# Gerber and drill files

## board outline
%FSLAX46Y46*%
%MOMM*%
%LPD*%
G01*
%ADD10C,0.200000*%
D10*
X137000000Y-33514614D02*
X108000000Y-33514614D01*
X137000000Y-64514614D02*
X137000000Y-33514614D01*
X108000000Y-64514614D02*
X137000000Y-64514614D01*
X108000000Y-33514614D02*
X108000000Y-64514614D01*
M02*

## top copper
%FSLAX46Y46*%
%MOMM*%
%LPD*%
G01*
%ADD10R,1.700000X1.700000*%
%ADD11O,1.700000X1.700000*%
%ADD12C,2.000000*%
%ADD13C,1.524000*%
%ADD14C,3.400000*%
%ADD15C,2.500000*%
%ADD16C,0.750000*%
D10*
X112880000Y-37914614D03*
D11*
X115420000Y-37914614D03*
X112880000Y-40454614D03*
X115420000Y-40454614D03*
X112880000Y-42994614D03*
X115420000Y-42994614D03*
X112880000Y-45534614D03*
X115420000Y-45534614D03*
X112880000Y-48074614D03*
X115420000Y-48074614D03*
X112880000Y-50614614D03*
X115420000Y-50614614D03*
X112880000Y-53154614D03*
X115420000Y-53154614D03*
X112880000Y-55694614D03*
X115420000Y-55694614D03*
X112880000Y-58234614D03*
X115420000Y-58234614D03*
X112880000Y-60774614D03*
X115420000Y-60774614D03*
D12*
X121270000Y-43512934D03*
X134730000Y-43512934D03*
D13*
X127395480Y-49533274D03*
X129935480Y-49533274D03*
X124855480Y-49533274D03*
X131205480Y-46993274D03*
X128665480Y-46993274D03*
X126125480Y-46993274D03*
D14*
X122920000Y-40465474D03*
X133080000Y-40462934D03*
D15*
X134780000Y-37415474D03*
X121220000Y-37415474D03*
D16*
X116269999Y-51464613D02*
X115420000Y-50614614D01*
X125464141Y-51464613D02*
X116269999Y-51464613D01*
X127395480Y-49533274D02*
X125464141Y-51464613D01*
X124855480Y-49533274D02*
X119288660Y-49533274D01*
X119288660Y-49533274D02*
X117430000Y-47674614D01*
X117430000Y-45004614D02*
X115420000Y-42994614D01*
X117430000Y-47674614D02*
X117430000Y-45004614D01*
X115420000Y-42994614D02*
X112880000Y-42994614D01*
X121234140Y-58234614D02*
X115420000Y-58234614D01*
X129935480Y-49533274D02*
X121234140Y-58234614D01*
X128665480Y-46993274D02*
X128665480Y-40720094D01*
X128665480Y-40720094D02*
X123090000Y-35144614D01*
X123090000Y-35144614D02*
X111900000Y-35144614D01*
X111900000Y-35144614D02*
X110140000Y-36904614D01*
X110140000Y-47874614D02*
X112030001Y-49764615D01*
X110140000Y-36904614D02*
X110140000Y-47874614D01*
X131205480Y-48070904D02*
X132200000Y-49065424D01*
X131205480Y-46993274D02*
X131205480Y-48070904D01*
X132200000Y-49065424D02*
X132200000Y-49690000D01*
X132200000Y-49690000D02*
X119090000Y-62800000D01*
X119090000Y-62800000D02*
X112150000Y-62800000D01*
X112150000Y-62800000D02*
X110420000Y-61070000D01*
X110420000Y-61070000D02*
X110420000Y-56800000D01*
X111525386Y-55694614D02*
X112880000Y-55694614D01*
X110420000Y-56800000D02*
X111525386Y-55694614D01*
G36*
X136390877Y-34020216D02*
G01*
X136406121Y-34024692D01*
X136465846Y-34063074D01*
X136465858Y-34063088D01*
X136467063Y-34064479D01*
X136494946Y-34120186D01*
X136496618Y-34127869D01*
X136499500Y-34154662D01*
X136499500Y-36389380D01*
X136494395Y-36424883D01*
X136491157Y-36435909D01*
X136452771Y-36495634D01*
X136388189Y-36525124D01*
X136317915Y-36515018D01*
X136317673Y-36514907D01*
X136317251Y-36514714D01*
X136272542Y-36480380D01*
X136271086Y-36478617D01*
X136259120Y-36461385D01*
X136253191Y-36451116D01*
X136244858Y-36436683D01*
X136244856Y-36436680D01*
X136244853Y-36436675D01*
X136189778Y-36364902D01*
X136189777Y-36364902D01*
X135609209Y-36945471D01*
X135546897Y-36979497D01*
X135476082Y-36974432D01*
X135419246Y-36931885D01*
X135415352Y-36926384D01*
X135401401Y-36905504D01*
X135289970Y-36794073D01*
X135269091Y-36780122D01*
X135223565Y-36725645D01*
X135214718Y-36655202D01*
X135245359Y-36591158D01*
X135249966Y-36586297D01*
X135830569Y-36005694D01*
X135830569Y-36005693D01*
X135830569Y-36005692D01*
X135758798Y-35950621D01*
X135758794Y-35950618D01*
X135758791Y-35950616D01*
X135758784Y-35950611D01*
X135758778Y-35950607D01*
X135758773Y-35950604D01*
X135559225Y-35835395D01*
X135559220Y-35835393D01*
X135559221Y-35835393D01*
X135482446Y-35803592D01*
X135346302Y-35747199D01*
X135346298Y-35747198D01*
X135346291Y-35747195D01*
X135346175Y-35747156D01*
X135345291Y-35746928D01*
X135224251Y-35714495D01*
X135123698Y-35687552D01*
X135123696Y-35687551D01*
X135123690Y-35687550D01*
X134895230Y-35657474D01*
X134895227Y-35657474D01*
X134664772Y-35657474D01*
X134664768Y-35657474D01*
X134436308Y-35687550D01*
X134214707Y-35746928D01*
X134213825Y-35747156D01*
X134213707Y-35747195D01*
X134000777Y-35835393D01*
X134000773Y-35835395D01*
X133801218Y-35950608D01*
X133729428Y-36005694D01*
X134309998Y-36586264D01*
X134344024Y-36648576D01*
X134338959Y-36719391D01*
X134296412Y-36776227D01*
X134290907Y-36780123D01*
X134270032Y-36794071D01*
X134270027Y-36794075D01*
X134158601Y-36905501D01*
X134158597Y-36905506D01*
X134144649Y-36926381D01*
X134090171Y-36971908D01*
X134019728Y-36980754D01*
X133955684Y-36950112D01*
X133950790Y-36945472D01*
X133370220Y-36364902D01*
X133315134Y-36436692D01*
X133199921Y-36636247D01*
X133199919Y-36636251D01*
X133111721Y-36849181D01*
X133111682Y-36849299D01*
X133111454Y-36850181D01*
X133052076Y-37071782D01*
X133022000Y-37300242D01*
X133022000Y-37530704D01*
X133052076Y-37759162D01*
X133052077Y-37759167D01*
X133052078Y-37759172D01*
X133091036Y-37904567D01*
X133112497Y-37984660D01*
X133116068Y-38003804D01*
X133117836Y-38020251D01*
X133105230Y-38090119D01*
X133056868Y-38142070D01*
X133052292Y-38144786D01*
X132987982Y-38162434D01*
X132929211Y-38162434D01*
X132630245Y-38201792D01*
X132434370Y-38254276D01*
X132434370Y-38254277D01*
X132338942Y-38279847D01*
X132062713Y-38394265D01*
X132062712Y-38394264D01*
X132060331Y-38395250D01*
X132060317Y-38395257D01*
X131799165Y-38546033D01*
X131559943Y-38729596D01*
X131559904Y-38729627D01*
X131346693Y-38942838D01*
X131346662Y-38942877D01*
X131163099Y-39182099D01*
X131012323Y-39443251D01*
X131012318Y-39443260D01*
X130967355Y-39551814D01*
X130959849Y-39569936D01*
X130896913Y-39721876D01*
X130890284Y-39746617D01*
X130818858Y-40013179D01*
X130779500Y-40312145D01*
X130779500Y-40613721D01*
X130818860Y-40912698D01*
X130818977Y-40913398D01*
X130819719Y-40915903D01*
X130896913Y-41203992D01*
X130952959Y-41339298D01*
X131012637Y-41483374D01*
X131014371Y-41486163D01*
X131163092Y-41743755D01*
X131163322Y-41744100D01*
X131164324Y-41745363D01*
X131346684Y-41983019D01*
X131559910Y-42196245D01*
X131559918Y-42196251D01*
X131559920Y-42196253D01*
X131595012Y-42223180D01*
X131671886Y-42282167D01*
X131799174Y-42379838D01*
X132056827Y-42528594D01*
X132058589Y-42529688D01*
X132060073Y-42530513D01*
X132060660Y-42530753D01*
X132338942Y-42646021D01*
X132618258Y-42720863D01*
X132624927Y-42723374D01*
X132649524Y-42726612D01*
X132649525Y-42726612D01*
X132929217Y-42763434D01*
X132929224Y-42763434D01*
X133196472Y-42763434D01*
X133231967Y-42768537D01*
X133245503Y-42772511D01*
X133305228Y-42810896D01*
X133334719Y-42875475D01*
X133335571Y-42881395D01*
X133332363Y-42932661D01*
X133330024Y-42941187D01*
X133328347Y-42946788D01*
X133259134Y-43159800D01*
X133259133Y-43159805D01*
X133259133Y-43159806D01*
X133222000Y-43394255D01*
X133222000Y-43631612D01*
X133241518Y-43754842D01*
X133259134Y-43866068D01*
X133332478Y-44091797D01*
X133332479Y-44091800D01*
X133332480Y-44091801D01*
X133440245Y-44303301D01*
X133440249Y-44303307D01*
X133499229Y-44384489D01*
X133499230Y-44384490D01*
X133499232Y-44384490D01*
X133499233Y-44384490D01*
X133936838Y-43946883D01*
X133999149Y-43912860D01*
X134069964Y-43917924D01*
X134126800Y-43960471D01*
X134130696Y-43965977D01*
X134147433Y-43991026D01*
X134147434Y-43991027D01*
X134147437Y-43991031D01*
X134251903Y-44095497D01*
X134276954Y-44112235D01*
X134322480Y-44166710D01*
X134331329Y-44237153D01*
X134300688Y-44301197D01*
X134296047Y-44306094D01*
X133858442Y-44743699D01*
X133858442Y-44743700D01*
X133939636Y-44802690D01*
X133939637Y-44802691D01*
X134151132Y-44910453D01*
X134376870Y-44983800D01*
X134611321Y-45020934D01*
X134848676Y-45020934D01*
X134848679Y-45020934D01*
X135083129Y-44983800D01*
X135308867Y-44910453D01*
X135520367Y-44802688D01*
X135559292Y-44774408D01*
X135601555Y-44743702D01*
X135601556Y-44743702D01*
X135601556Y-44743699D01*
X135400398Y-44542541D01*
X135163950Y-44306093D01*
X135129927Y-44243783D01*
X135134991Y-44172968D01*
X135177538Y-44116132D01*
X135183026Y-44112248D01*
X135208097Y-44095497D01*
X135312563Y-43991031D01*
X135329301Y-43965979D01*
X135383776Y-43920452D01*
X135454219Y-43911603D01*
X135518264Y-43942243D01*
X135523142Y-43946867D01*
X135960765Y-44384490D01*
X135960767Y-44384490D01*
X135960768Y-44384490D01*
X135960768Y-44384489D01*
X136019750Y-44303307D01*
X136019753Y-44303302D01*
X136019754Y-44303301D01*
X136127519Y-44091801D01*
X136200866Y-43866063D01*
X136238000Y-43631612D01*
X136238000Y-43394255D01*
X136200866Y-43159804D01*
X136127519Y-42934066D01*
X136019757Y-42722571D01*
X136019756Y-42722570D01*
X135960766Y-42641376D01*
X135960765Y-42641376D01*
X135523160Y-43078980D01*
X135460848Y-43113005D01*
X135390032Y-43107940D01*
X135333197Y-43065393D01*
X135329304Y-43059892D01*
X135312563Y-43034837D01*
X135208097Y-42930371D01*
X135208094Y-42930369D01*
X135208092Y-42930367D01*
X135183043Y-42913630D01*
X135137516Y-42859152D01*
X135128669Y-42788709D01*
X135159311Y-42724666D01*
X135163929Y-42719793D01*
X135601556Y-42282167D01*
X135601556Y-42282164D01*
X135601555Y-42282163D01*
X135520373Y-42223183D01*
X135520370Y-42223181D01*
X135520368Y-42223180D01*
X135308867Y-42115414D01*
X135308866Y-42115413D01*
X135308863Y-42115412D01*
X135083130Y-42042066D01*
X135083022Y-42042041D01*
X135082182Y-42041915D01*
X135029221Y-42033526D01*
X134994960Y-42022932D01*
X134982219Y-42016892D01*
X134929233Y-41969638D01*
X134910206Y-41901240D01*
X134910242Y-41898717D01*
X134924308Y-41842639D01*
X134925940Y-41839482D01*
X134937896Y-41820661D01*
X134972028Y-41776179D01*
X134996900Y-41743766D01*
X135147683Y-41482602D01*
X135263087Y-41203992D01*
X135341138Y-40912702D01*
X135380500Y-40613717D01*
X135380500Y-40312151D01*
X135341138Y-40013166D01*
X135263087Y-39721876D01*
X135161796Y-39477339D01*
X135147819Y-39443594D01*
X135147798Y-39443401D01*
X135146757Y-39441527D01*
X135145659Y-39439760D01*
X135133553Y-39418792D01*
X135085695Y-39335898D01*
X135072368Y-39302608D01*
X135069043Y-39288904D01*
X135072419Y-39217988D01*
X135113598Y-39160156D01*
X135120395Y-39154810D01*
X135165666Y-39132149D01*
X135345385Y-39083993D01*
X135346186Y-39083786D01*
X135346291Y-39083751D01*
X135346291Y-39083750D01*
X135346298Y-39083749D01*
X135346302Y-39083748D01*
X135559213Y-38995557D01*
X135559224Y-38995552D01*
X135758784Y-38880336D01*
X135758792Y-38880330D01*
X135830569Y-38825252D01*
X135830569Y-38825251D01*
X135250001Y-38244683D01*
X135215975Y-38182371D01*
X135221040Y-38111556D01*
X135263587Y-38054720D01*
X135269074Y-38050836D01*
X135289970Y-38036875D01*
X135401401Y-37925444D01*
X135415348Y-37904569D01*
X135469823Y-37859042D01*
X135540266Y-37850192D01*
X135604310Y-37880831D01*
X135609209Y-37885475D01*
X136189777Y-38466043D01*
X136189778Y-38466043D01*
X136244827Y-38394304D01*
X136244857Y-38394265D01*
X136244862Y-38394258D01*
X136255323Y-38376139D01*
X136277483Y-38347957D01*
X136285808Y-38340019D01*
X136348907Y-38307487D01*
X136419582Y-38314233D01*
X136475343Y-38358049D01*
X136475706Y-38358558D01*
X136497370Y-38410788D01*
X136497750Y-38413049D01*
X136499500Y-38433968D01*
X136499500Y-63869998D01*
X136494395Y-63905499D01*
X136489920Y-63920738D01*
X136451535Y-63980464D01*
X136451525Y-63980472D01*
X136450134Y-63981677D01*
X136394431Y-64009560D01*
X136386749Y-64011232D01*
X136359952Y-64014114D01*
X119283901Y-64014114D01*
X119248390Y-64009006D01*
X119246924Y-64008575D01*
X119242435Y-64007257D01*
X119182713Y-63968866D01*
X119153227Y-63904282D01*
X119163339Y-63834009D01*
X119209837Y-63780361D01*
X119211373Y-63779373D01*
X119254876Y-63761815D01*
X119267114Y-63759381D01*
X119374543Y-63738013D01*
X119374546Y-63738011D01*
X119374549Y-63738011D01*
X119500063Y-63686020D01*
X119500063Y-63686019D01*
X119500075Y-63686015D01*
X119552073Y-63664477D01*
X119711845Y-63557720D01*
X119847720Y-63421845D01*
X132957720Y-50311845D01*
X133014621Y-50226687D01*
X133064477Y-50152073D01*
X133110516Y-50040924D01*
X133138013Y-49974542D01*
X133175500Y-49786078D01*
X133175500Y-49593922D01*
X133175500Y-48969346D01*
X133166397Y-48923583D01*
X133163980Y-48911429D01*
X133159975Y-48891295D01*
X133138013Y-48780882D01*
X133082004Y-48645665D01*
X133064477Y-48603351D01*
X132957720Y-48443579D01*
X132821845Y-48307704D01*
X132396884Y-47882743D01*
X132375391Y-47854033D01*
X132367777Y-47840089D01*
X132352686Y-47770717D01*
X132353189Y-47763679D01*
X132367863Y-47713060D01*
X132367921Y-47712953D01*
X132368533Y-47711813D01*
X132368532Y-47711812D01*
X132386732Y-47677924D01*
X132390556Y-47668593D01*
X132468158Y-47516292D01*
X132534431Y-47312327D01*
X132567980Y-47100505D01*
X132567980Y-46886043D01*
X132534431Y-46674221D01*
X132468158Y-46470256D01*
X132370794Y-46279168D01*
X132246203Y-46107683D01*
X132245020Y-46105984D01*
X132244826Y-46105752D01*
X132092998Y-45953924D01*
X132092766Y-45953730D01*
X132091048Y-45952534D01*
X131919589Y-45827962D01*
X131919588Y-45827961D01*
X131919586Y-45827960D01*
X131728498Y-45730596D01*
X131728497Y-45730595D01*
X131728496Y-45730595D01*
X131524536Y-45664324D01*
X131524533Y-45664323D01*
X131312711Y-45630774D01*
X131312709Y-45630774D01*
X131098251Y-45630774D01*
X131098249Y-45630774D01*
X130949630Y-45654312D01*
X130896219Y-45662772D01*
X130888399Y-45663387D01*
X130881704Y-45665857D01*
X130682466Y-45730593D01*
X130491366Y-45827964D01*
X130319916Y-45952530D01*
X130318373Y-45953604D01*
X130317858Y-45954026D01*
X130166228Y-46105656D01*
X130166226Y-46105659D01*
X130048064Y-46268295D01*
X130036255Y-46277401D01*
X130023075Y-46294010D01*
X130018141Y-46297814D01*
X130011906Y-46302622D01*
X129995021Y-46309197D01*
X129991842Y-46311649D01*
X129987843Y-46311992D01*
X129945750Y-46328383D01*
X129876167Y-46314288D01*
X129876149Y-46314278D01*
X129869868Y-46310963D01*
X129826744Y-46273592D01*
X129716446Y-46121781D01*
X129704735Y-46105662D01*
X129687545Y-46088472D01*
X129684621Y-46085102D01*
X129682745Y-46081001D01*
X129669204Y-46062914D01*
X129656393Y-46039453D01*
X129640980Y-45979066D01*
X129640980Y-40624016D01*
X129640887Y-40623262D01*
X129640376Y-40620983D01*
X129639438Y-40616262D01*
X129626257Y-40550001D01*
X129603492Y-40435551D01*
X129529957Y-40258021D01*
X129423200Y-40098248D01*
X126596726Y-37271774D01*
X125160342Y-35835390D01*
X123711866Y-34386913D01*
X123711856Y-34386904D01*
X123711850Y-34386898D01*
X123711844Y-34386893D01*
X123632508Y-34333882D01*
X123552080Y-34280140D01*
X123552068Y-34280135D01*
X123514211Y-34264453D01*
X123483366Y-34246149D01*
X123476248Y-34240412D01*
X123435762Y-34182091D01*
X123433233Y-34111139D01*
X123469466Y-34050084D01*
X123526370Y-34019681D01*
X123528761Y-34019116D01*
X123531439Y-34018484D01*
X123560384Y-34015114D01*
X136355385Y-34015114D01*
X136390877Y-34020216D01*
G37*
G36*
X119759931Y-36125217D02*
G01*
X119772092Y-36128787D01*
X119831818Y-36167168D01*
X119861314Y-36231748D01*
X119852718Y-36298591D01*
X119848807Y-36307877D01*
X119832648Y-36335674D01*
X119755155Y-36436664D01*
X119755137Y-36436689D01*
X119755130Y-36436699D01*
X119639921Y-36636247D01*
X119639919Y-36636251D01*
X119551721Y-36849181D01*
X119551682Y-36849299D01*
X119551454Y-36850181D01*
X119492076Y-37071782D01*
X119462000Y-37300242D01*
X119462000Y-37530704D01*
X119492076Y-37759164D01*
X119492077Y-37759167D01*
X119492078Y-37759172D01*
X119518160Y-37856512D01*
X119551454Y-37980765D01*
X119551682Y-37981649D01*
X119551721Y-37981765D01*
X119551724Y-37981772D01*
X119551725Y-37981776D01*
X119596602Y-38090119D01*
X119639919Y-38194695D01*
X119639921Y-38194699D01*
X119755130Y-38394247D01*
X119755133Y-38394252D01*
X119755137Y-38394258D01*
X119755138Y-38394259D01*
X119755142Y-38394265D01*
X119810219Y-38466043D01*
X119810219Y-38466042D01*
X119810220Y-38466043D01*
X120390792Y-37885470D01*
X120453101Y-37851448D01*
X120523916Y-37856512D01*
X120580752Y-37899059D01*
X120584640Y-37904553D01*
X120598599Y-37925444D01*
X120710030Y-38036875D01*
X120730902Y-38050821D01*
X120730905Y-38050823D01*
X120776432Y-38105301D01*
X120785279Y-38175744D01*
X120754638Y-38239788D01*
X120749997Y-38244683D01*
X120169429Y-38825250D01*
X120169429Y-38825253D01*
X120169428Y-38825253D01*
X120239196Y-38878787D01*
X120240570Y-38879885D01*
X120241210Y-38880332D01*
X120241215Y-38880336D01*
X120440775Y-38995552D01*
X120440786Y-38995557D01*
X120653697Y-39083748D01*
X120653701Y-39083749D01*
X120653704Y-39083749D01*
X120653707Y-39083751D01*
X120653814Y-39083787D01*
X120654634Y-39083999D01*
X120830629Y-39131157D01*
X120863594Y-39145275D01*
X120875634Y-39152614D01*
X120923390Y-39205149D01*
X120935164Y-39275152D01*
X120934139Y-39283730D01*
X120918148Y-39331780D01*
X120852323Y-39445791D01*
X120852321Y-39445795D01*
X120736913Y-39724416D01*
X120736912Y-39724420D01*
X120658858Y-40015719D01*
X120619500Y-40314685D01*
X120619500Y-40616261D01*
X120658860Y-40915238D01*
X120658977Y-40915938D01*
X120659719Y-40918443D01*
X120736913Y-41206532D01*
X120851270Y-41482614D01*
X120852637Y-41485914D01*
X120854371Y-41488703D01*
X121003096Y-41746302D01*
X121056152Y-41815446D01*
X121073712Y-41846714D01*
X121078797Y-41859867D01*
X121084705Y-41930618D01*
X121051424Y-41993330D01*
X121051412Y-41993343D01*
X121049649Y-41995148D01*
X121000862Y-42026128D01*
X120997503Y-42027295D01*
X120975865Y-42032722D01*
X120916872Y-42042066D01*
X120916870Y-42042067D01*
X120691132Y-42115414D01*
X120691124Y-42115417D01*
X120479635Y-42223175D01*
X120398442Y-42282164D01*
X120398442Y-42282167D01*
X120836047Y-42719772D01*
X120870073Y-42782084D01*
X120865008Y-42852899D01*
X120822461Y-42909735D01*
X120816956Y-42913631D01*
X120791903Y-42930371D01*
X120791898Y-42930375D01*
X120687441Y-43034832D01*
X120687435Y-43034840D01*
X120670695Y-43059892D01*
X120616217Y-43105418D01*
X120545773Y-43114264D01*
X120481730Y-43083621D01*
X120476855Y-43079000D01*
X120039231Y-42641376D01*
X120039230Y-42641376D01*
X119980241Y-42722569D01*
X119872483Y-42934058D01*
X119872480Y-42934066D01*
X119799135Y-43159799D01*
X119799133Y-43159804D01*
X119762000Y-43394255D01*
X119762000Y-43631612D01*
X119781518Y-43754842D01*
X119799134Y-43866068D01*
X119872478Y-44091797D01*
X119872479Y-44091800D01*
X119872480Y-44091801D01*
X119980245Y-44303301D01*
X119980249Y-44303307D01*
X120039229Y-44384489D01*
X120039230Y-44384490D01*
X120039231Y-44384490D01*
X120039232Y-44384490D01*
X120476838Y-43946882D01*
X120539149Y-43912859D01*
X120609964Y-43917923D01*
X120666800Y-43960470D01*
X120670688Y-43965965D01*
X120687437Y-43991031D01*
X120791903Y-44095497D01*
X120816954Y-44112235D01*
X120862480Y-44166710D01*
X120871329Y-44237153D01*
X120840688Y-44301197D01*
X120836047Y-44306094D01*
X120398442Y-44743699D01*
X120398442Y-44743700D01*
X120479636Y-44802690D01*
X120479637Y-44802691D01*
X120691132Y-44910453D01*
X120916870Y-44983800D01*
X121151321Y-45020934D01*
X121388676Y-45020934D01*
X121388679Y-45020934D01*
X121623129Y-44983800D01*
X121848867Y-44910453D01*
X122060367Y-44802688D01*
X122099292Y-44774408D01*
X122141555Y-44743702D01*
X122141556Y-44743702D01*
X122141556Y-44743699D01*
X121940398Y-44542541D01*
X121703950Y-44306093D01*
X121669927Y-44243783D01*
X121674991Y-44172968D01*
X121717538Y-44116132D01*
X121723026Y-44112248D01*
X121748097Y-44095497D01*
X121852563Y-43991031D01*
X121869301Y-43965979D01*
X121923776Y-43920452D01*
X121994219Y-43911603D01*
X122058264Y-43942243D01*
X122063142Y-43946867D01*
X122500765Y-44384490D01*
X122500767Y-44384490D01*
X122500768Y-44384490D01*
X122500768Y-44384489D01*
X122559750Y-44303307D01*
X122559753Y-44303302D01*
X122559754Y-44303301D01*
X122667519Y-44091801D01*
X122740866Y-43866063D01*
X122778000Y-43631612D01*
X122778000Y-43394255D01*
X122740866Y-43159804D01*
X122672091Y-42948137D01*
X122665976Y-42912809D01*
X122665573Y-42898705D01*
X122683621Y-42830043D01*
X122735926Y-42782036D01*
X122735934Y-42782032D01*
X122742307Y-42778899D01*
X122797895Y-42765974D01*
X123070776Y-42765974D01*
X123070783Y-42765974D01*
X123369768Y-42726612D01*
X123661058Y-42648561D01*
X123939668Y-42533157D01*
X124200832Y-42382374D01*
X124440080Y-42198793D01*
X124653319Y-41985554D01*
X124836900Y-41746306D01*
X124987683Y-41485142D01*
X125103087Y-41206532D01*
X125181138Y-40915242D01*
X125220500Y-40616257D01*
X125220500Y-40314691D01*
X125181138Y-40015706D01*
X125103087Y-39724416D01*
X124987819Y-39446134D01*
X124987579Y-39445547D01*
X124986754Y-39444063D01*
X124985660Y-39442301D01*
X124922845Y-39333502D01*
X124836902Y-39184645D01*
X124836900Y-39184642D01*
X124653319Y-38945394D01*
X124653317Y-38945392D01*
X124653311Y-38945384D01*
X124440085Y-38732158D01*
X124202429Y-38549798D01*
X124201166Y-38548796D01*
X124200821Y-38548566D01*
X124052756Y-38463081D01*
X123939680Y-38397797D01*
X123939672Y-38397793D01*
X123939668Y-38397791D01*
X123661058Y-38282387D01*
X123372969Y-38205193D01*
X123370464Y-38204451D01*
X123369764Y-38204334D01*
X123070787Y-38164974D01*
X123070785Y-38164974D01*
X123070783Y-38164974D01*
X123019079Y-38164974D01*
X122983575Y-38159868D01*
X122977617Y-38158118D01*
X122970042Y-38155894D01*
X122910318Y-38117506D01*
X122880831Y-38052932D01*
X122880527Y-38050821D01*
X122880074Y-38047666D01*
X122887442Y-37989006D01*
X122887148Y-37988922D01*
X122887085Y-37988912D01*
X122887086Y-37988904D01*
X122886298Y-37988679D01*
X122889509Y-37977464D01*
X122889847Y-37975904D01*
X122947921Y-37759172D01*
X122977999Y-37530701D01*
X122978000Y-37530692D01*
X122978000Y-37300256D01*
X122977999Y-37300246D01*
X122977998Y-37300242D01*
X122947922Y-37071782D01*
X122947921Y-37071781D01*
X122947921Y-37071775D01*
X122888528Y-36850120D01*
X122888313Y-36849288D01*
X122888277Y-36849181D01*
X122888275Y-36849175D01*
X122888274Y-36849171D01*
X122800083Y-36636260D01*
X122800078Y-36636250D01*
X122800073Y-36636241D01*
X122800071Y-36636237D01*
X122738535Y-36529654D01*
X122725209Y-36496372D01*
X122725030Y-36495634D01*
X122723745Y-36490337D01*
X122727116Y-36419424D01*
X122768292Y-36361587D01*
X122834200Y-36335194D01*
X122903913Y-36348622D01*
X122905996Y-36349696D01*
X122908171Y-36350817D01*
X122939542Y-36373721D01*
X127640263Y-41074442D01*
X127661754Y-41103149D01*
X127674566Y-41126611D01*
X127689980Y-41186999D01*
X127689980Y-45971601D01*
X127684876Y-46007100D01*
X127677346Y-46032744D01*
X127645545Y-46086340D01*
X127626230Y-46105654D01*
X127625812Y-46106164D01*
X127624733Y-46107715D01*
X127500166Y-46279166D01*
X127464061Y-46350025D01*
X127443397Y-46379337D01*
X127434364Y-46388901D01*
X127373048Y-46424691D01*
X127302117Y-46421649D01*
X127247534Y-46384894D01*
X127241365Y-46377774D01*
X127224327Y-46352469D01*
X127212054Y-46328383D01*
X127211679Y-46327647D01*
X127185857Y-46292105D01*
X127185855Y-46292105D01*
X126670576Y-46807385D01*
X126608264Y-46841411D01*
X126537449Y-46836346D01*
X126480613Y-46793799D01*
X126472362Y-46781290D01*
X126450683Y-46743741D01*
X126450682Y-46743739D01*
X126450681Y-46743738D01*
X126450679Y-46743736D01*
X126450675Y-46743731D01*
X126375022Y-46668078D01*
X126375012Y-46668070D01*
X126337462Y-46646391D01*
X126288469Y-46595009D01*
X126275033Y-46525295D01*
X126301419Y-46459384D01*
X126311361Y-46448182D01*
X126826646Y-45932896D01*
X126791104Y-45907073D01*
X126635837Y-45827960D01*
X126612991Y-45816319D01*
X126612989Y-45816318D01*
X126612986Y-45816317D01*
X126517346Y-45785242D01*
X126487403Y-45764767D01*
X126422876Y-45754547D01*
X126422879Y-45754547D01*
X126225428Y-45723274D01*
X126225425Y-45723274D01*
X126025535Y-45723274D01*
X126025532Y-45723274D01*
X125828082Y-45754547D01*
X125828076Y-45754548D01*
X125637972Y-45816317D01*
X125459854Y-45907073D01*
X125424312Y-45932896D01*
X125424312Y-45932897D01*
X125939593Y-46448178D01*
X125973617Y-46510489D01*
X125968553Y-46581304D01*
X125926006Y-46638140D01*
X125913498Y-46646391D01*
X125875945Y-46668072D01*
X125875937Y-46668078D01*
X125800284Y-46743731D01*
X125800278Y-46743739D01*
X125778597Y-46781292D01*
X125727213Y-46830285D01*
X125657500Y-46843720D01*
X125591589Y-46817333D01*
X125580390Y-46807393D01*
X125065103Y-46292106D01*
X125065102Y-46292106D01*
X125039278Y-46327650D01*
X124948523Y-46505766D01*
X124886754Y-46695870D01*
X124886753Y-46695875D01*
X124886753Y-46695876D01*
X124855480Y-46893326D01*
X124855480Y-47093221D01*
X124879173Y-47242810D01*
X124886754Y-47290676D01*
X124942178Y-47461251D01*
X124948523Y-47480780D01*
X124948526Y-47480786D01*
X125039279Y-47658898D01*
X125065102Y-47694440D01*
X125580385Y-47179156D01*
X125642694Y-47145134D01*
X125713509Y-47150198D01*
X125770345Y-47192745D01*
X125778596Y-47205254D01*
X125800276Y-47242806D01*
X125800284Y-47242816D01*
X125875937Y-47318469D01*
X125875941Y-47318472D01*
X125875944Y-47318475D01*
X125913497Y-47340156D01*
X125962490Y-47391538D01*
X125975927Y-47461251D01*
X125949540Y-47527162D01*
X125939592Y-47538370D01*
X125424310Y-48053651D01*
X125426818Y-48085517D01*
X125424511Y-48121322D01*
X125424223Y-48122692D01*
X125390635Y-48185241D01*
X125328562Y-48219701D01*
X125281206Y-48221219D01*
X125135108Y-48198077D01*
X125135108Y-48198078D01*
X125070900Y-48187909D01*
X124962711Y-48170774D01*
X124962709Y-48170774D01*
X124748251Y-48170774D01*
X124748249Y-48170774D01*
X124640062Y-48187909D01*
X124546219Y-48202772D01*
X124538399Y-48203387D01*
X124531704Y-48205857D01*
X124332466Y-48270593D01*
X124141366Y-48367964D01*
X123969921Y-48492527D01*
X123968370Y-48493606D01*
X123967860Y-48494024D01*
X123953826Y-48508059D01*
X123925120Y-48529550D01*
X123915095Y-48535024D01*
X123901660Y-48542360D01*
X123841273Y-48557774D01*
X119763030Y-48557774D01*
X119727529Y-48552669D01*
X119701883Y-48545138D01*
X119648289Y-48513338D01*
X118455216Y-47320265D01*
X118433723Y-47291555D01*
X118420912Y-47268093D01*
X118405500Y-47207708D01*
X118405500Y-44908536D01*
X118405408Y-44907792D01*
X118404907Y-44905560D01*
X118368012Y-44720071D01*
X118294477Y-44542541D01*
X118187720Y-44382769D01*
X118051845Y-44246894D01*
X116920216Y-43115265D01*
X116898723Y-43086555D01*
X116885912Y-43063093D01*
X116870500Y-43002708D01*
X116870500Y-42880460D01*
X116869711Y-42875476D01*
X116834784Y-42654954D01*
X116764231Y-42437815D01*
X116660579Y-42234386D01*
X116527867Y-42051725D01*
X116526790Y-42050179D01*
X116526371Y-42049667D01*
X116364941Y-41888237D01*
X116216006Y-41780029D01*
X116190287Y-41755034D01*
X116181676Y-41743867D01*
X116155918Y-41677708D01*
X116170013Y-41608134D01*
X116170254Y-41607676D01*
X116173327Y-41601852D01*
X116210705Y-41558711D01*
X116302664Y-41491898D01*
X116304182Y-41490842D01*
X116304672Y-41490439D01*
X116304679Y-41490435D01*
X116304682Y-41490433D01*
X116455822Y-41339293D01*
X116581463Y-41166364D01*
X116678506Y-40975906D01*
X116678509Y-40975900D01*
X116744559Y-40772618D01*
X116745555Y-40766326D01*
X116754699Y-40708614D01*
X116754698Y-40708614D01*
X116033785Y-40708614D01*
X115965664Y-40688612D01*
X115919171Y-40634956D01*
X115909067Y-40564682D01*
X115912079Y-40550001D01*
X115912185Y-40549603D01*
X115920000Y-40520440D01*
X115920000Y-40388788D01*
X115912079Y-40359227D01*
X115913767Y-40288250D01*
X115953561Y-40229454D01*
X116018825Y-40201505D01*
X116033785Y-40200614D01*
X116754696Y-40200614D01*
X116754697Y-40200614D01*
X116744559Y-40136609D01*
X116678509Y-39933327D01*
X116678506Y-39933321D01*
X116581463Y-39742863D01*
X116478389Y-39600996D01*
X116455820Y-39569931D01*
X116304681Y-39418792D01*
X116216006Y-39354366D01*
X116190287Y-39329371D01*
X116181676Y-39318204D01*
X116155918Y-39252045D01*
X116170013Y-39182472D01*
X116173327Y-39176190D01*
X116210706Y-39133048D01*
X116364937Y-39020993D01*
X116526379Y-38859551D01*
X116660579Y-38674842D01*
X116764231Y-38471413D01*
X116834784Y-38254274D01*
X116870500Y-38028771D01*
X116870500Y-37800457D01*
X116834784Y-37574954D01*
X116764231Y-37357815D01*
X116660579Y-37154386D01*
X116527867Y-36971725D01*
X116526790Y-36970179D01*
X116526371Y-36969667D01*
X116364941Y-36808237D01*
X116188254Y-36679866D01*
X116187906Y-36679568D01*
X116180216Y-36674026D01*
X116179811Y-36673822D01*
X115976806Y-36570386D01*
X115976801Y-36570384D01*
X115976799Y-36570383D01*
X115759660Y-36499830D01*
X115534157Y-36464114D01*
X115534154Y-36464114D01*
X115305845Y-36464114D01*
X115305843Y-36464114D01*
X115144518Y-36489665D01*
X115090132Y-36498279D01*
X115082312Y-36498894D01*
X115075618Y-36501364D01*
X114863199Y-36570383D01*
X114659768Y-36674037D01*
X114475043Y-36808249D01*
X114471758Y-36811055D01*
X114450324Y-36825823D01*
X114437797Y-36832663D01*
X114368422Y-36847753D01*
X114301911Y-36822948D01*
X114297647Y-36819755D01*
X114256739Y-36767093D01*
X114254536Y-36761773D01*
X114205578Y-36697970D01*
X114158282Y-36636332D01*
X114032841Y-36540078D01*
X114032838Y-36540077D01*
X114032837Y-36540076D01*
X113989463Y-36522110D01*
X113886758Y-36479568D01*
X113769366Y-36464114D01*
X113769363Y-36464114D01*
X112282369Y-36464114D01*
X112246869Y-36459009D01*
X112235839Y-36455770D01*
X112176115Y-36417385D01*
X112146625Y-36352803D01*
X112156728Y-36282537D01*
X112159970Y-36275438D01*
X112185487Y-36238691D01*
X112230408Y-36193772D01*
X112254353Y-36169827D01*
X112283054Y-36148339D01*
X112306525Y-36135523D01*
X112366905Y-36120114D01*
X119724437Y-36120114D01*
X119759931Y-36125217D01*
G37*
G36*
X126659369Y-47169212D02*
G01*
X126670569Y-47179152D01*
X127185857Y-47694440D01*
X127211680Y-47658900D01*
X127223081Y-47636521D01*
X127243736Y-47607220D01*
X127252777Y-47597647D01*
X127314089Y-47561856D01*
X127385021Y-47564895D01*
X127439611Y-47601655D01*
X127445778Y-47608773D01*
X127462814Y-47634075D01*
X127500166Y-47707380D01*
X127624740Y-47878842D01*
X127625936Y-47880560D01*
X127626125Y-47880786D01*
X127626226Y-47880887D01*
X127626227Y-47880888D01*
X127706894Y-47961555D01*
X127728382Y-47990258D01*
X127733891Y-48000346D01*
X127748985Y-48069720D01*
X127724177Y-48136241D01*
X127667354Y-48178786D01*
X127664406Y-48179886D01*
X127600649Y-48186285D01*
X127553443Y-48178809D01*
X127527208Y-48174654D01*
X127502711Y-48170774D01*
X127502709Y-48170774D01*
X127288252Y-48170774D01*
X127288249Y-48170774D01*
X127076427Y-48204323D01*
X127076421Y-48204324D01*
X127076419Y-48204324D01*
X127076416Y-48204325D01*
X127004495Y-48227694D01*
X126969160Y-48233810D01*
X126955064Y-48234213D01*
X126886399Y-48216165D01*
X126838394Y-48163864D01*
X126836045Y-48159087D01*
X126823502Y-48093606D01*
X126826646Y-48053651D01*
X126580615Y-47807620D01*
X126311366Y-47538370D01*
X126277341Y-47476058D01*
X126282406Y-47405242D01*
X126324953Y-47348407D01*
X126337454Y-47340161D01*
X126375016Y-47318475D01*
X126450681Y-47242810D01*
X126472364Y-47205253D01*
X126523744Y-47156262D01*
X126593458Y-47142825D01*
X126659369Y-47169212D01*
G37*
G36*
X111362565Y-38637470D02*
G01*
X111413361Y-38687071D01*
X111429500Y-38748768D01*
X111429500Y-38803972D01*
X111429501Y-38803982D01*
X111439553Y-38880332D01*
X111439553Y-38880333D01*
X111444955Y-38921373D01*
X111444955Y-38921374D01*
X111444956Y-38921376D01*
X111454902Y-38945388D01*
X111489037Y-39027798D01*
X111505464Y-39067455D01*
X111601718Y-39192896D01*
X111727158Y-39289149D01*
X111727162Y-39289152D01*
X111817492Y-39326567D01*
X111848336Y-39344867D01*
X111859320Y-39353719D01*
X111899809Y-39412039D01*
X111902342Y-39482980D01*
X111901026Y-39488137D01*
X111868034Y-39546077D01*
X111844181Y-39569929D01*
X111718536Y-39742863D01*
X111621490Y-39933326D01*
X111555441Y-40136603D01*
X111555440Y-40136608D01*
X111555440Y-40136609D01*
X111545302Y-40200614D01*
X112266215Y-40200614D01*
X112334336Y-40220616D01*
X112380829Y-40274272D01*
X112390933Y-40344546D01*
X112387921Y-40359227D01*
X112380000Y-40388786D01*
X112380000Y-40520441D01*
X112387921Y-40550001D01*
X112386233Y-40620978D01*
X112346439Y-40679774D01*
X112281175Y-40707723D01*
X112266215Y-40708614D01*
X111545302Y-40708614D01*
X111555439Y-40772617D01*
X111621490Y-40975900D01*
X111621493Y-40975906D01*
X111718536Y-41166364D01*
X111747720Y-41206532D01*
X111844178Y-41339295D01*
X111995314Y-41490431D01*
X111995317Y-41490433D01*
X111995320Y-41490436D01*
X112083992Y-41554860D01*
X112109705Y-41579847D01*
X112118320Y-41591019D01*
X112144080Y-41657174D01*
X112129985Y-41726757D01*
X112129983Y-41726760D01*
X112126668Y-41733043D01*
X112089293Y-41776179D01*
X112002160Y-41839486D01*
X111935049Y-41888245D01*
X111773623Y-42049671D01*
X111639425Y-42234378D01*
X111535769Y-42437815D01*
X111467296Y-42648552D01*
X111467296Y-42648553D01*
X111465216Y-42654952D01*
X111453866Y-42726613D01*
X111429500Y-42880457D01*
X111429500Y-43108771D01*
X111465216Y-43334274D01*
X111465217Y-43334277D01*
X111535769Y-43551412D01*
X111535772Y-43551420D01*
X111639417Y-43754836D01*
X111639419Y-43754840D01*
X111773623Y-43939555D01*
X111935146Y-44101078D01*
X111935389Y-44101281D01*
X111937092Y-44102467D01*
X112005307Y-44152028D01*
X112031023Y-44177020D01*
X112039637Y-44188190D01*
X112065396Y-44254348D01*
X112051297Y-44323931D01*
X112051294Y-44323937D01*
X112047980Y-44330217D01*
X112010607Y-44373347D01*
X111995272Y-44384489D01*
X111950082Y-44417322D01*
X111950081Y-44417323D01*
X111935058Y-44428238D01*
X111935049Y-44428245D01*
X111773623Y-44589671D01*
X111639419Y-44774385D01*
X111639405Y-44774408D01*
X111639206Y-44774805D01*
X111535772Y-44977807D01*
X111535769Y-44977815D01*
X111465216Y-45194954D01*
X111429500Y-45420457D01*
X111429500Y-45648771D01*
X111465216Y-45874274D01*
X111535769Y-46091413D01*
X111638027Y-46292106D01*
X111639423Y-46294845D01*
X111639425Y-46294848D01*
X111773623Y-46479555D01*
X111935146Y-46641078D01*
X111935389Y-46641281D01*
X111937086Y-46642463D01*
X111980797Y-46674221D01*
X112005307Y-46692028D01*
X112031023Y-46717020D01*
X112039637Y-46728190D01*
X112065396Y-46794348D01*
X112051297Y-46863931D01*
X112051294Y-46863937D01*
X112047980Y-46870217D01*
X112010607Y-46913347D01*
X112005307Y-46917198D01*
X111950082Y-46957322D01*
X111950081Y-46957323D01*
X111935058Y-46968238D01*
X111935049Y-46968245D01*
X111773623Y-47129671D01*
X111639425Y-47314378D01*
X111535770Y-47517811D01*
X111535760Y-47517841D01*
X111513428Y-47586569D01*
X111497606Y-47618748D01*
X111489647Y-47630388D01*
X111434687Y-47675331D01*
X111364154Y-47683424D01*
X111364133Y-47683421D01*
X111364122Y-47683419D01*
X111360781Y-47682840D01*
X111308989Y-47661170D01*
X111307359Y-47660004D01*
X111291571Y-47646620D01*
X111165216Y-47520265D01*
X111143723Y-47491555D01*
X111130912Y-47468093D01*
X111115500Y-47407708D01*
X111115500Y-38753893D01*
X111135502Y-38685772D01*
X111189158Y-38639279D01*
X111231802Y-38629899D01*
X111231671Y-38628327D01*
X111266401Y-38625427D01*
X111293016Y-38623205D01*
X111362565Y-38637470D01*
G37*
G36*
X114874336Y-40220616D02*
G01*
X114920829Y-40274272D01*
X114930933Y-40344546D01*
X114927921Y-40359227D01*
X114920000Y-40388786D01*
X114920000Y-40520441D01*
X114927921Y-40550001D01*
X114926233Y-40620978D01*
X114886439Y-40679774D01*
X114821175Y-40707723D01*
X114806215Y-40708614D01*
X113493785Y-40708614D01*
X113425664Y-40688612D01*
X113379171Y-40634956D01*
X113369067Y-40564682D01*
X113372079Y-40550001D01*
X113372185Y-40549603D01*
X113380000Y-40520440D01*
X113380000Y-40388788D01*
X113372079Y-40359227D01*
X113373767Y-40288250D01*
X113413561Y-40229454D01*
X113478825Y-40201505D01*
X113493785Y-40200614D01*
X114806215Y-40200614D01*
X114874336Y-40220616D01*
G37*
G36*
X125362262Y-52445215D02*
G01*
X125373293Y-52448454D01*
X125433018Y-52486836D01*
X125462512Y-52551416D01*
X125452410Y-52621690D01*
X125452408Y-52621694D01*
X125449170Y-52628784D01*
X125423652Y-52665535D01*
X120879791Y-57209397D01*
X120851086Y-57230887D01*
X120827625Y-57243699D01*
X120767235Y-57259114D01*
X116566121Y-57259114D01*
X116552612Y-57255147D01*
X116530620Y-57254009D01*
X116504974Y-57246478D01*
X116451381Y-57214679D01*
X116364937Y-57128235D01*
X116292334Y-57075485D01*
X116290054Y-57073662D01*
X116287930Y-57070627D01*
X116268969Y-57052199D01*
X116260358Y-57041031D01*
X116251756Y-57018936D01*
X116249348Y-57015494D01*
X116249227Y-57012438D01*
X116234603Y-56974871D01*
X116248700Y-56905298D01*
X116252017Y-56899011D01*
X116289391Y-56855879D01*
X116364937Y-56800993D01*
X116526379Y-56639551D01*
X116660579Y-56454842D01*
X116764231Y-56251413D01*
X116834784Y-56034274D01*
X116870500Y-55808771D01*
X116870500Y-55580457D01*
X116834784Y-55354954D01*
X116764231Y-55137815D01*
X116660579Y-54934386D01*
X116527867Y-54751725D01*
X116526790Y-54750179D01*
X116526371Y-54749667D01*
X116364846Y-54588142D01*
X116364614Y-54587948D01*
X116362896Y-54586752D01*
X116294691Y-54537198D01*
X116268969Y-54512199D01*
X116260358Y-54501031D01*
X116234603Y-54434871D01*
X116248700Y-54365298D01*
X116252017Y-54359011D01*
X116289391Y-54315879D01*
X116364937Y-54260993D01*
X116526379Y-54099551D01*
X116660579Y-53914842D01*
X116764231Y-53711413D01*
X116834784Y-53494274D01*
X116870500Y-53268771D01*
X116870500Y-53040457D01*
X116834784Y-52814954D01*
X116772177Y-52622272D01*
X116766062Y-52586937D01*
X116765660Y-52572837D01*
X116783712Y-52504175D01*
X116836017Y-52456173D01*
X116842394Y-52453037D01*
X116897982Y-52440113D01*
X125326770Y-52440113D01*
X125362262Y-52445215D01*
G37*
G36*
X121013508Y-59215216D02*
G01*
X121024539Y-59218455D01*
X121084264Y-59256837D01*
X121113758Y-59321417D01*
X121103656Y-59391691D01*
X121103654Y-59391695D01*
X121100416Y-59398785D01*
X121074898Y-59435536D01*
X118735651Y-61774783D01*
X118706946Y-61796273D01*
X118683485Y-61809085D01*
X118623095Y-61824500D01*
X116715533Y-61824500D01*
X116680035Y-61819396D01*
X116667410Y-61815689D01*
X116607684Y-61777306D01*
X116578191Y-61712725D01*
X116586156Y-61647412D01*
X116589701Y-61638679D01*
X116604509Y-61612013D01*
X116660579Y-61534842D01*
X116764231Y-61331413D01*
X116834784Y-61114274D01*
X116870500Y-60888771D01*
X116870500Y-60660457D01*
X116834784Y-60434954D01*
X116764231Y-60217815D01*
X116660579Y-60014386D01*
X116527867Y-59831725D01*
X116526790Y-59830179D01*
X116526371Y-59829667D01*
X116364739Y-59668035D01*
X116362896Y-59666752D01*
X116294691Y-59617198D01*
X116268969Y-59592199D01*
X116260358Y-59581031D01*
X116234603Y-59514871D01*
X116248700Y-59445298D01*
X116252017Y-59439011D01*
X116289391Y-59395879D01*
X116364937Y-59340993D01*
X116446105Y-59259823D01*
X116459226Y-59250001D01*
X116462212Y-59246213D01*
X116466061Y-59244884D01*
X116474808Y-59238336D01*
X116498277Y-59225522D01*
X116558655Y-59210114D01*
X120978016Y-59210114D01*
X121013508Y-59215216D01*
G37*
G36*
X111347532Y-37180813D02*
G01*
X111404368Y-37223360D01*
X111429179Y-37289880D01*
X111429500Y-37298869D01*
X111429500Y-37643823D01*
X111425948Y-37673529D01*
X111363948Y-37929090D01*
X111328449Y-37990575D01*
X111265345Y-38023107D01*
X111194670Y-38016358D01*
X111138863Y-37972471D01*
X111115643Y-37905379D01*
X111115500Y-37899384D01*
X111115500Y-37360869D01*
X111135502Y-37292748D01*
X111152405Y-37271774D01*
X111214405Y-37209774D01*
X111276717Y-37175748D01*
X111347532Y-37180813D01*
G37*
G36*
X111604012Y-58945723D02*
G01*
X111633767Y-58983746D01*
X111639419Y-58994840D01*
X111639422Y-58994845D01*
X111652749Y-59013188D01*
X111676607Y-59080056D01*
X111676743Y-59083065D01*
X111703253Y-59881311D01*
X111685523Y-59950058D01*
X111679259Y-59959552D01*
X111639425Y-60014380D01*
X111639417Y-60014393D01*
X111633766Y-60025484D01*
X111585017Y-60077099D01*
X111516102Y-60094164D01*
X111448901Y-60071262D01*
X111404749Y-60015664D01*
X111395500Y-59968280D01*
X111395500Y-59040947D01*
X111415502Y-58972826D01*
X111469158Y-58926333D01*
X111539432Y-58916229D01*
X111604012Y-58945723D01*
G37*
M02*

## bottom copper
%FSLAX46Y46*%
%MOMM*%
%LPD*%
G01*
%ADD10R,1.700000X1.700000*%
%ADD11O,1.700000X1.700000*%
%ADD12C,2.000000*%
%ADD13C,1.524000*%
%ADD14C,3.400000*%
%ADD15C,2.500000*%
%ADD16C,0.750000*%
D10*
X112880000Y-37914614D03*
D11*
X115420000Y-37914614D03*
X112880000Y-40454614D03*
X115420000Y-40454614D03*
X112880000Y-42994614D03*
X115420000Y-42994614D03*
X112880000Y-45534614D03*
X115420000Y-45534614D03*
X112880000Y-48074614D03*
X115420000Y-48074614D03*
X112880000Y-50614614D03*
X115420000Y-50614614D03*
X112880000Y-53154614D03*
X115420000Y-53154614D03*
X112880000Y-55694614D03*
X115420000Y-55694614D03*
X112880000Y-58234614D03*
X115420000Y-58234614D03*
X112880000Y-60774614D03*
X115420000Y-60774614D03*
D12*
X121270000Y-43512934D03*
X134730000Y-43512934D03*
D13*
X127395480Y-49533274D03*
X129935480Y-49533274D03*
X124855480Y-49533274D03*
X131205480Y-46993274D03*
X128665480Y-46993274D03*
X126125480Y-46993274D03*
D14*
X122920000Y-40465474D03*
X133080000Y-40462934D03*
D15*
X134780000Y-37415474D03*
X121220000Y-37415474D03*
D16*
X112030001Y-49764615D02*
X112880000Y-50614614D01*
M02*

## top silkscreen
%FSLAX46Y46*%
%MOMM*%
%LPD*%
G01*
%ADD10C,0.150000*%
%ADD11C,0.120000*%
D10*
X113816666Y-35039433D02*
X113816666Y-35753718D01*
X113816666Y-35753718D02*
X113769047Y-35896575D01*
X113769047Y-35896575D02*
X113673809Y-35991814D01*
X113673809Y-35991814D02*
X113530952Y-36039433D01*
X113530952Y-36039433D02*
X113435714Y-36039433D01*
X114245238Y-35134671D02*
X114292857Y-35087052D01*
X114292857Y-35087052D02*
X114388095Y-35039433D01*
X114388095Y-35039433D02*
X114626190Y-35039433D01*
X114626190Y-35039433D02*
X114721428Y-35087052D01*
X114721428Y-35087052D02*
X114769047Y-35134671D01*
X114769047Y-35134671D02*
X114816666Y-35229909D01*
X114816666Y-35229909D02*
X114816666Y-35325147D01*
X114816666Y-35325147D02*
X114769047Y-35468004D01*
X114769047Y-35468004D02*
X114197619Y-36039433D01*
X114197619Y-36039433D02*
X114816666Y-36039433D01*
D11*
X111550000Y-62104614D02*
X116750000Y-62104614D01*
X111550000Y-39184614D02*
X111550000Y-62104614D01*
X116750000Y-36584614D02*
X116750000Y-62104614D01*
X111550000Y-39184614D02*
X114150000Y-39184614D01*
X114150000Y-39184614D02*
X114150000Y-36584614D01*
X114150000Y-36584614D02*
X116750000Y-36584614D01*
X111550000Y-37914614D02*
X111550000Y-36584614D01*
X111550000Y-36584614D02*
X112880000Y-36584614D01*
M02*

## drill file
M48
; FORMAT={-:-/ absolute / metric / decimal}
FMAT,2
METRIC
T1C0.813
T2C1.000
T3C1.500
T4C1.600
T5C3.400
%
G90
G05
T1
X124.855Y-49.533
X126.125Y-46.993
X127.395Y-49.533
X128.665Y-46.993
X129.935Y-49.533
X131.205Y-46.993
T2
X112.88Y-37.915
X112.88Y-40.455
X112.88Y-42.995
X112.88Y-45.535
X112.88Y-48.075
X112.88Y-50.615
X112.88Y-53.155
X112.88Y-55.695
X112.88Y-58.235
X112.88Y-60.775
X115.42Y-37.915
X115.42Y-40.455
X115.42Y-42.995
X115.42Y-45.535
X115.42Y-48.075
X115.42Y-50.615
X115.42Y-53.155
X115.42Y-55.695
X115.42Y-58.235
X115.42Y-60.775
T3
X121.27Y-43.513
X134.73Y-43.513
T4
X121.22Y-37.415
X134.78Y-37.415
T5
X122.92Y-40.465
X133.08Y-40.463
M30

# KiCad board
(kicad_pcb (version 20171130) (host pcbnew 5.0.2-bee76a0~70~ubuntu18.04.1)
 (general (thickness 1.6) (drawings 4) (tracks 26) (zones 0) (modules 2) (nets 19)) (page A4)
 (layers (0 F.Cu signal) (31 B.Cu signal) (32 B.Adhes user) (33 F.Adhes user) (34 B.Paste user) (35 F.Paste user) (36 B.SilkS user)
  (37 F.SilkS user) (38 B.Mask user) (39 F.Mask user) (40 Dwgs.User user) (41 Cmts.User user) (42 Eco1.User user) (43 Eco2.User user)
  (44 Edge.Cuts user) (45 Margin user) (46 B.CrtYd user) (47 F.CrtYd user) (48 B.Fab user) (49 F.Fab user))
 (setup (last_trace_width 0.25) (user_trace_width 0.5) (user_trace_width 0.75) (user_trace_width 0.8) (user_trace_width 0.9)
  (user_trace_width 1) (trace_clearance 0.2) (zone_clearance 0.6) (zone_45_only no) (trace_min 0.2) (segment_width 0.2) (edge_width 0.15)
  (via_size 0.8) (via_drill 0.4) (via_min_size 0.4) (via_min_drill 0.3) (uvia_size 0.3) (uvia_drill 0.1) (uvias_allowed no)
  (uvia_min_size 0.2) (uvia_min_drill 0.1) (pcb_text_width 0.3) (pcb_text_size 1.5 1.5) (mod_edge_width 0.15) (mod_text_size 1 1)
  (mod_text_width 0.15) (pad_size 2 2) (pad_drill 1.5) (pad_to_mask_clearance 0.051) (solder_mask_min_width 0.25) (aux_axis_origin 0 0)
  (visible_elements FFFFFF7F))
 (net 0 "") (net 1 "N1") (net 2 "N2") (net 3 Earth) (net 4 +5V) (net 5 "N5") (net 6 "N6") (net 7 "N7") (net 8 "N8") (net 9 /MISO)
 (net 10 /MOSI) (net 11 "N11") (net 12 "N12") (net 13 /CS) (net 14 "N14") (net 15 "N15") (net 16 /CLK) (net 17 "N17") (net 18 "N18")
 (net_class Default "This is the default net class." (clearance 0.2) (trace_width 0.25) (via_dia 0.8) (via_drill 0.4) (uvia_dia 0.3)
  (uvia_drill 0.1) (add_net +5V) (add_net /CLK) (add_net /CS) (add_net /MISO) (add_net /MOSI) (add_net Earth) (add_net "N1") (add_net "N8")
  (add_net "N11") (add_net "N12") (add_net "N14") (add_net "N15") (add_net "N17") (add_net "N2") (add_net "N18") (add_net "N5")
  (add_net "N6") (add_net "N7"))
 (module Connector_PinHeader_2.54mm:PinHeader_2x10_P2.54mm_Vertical (layer F.Cu) (at 112.88 37.914614)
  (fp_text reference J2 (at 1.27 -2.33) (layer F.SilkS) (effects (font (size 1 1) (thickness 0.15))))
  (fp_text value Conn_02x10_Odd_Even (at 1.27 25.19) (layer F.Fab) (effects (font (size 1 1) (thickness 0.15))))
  (fp_line (start -1.33 24.19) (end 3.87 24.19) (layer F.SilkS) (width 0.12))
  (fp_line (start -1.33 1.27) (end -1.33 24.19) (layer F.SilkS) (width 0.12))
  (fp_line (start 3.87 -1.33) (end 3.87 24.19) (layer F.SilkS) (width 0.12))
  (fp_line (start -1.33 1.27) (end 1.27 1.27) (layer F.SilkS) (width 0.12))
  (fp_line (start 1.27 1.27) (end 1.27 -1.33) (layer F.SilkS) (width 0.12))
  (fp_line (start 1.27 -1.33) (end 3.87 -1.33) (layer F.SilkS) (width 0.12))
  (fp_line (start -1.33 0) (end -1.33 -1.33) (layer F.SilkS) (width 0.12))
  (fp_line (start -1.33 -1.33) (end 0 -1.33) (layer F.SilkS) (width 0.12))
  (pad 1 thru_hole rect (at 0 0) (size 1.7 1.7) (drill 1) (layers *.Cu *.Mask) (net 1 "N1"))
  (pad 2 thru_hole oval (at 2.54 0) (size 1.7 1.7) (drill 1) (layers *.Cu *.Mask) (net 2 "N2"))
  (pad 3 thru_hole oval (at 0 2.54) (size 1.7 1.7) (drill 1) (layers *.Cu *.Mask) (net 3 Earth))
  (pad 4 thru_hole oval (at 2.54 2.54) (size 1.7 1.7) (drill 1) (layers *.Cu *.Mask) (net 3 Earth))
  (pad 5 thru_hole oval (at 0 5.08) (size 1.7 1.7) (drill 1) (layers *.Cu *.Mask) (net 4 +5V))
  (pad 6 thru_hole oval (at 2.54 5.08) (size 1.7 1.7) (drill 1) (layers *.Cu *.Mask) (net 4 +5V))
  (pad 7 thru_hole oval (at 0 7.62) (size 1.7 1.7) (drill 1) (layers *.Cu *.Mask) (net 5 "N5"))
  (pad 8 thru_hole oval (at 2.54 7.62) (size 1.7 1.7) (drill 1) (layers *.Cu *.Mask) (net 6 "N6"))
  (pad 9 thru_hole oval (at 0 10.16) (size 1.7 1.7) (drill 1) (layers *.Cu *.Mask) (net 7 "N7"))
  (pad 10 thru_hole oval (at 2.54 10.16) (size 1.7 1.7) (drill 1) (layers *.Cu *.Mask) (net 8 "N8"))
  (pad 11 thru_hole oval (at 0 12.7) (size 1.7 1.7) (drill 1) (layers *.Cu *.Mask) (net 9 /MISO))
  (pad 12 thru_hole oval (at 2.54 12.7) (size 1.7 1.7) (drill 1) (layers *.Cu *.Mask) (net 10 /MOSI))
  (pad 13 thru_hole oval (at 0 15.24) (size 1.7 1.7) (drill 1) (layers *.Cu *.Mask) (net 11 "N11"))
  (pad 14 thru_hole oval (at 2.54 15.24) (size 1.7 1.7) (drill 1) (layers *.Cu *.Mask) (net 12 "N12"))
  (pad 15 thru_hole oval (at 0 17.78) (size 1.7 1.7) (drill 1) (layers *.Cu *.Mask) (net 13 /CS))
  (pad 16 thru_hole oval (at 2.54 17.78) (size 1.7 1.7) (drill 1) (layers *.Cu *.Mask) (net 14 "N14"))
  (pad 17 thru_hole oval (at 0 20.32) (size 1.7 1.7) (drill 1) (layers *.Cu *.Mask) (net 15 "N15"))
  (pad 18 thru_hole oval (at 2.54 20.32) (size 1.7 1.7) (drill 1) (layers *.Cu *.Mask) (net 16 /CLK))
  (pad 19 thru_hole oval (at 0 22.86) (size 1.7 1.7) (drill 1) (layers *.Cu *.Mask) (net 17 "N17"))
  (pad 20 thru_hole oval (at 2.54 22.86) (size 1.7 1.7) (drill 1) (layers *.Cu *.Mask) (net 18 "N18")))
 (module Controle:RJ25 (layer B.Cu) (at 128 45.014614)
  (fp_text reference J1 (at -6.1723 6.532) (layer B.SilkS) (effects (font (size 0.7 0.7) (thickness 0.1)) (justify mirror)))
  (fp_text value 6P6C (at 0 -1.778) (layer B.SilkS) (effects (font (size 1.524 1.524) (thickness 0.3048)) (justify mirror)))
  (pad 0 thru_hole circle (at -6.73 -1.50168 180) (size 2 2) (drill 1.5) (layers *.Cu *.Mask F.Adhes B.SilkS) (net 3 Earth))
  (pad 0 thru_hole circle (at 6.73 -1.50168 180) (size 2 2) (drill 1.5) (layers *.Cu *.Mask B.SilkS) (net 3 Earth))
  (pad 3 thru_hole circle (at -0.60452 4.51866 180) (size 1.524 1.524) (drill 0.8128) (layers *.Cu *.Mask B.SilkS) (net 10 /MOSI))
  (pad 5 thru_hole circle (at 1.93548 4.51866 180) (size 1.524 1.524) (drill 0.8128) (layers *.Cu *.Mask B.SilkS) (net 16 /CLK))
  (pad 1 thru_hole circle (at -3.14452 4.51866 180) (size 1.524 1.524) (drill 0.8128) (layers *.Cu *.Mask B.SilkS) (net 4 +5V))
  (pad 6 thru_hole circle (at 3.20548 1.97866 180) (size 1.524 1.524) (drill 0.8128) (layers *.Cu *.Mask B.SilkS) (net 13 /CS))
  (pad 4 thru_hole circle (at 0.66548 1.97866 180) (size 1.524 1.524) (drill 0.8128) (layers *.Cu *.Mask B.SilkS) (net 9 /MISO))
  (pad 2 thru_hole circle (at -1.87452 1.97866 180) (size 1.524 1.524) (drill 0.8128) (layers *.Cu *.Mask B.SilkS) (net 3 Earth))
  (pad 0 thru_hole circle (at -5.08 -4.54914 180) (size 3.4 3.4) (drill 3.4) (layers *.Cu *.Mask B.SilkS))
  (pad 0 thru_hole circle (at 5.08 -4.55168 180) (size 3.4 3.4) (drill 3.4) (layers *.Cu *.Mask B.SilkS))
  (pad 0 thru_hole circle (at 6.78 -7.59914 180) (size 2.5 2.5) (drill 1.6) (layers *.Cu *.Mask B.SilkS) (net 3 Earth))
  (pad 0 thru_hole circle (at -6.78 -7.59914 180) (size 2.5 2.5) (drill 1.6) (layers *.Cu *.Mask B.SilkS) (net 3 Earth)))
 (gr_line (start 137 33.514614) (end 108 33.514614) (layer Edge.Cuts) (width 0.2))
 (gr_line (start 137 64.514614) (end 137 33.514614) (layer Edge.Cuts) (width 0.2))
 (gr_line (start 108 64.514614) (end 137 64.514614) (layer Edge.Cuts) (width 0.2))
 (gr_line (start 108 33.514614) (end 108 64.514614) (layer Edge.Cuts) (width 0.2))
 (segment (start 116.269999 51.464613) (end 115.42 50.614614) (width 0.75) (layer F.Cu) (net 10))
 (segment (start 125.464141 51.464613) (end 116.269999 51.464613) (width 0.75) (layer F.Cu) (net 10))
 (segment (start 127.39548 49.533274) (end 125.464141 51.464613) (width 0.75) (layer F.Cu) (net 10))
 (segment (start 124.85548 49.533274) (end 119.28866 49.533274) (width 0.75) (layer F.Cu) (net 4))
 (segment (start 119.28866 49.533274) (end 117.43 47.674614) (width 0.75) (layer F.Cu) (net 4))
 (segment (start 117.43 45.004614) (end 115.42 42.994614) (width 0.75) (layer F.Cu) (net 4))
 (segment (start 117.43 47.674614) (end 117.43 45.004614) (width 0.75) (layer F.Cu) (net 4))
 (segment (start 115.42 42.994614) (end 112.88 42.994614) (width 0.75) (layer F.Cu) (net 4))
 (segment (start 121.23414 58.234614) (end 115.42 58.234614) (width 0.75) (layer F.Cu) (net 16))
 (segment (start 129.93548 49.533274) (end 121.23414 58.234614) (width 0.75) (layer F.Cu) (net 16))
 (segment (start 128.66548 46.993274) (end 128.66548 40.720094) (width 0.75) (layer F.Cu) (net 9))
 (segment (start 128.66548 40.720094) (end 123.09 35.144614) (width 0.75) (layer F.Cu) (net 9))
 (segment (start 123.09 35.144614) (end 111.9 35.144614) (width 0.75) (layer F.Cu) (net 9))
 (segment (start 111.9 35.144614) (end 110.14 36.904614) (width 0.75) (layer F.Cu) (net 9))
 (segment (start 112.030001 49.764615) (end 112.88 50.614614) (width 0.75) (layer B.Cu) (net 9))
 (segment (start 110.14 47.874614) (end 112.030001 49.764615) (width 0.75) (layer F.Cu) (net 9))
 (segment (start 110.14 36.904614) (end 110.14 47.874614) (width 0.75) (layer F.Cu) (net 9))
 (segment (start 131.20548 48.070904) (end 132.2 49.065424) (width 0.75) (layer F.Cu) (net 13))
 (segment (start 131.20548 46.993274) (end 131.20548 48.070904) (width 0.75) (layer F.Cu) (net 13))
 (segment (start 132.2 49.065424) (end 132.2 49.69) (width 0.75) (layer F.Cu) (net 13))
 (segment (start 132.2 49.69) (end 119.09 62.8) (width 0.75) (layer F.Cu) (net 13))
 (segment (start 119.09 62.8) (end 112.15 62.8) (width 0.75) (layer F.Cu) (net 13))
 (segment (start 112.15 62.8) (end 110.42 61.07) (width 0.75) (layer F.Cu) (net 13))
 (segment (start 110.42 61.07) (end 110.42 56.8) (width 0.75) (layer F.Cu) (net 13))
 (segment (start 111.525386 55.694614) (end 112.88 55.694614) (width 0.75) (layer F.Cu) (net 13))
 (segment (start 110.42 56.8) (end 111.525386 55.694614) (width 0.75) (layer F.Cu) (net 13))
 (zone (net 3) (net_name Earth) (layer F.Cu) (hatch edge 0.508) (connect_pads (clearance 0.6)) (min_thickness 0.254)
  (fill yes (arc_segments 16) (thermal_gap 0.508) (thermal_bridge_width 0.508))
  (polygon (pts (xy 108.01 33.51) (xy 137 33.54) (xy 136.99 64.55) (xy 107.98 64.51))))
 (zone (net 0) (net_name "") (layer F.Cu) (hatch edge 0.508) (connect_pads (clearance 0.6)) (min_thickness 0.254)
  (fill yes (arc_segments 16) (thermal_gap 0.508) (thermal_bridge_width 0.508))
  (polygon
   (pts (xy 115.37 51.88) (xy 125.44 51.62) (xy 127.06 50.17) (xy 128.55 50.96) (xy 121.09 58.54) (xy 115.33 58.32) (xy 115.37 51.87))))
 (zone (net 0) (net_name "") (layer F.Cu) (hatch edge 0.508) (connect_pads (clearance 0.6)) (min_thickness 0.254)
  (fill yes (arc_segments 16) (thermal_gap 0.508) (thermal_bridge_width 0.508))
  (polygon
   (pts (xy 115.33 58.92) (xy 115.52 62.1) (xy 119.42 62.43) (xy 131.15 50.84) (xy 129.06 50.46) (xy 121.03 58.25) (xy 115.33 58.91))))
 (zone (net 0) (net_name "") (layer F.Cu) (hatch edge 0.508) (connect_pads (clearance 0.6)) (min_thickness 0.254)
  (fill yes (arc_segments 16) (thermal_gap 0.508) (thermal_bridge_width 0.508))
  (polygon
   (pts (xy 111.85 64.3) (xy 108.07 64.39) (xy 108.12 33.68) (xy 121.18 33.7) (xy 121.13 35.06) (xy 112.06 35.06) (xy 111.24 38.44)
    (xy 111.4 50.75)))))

